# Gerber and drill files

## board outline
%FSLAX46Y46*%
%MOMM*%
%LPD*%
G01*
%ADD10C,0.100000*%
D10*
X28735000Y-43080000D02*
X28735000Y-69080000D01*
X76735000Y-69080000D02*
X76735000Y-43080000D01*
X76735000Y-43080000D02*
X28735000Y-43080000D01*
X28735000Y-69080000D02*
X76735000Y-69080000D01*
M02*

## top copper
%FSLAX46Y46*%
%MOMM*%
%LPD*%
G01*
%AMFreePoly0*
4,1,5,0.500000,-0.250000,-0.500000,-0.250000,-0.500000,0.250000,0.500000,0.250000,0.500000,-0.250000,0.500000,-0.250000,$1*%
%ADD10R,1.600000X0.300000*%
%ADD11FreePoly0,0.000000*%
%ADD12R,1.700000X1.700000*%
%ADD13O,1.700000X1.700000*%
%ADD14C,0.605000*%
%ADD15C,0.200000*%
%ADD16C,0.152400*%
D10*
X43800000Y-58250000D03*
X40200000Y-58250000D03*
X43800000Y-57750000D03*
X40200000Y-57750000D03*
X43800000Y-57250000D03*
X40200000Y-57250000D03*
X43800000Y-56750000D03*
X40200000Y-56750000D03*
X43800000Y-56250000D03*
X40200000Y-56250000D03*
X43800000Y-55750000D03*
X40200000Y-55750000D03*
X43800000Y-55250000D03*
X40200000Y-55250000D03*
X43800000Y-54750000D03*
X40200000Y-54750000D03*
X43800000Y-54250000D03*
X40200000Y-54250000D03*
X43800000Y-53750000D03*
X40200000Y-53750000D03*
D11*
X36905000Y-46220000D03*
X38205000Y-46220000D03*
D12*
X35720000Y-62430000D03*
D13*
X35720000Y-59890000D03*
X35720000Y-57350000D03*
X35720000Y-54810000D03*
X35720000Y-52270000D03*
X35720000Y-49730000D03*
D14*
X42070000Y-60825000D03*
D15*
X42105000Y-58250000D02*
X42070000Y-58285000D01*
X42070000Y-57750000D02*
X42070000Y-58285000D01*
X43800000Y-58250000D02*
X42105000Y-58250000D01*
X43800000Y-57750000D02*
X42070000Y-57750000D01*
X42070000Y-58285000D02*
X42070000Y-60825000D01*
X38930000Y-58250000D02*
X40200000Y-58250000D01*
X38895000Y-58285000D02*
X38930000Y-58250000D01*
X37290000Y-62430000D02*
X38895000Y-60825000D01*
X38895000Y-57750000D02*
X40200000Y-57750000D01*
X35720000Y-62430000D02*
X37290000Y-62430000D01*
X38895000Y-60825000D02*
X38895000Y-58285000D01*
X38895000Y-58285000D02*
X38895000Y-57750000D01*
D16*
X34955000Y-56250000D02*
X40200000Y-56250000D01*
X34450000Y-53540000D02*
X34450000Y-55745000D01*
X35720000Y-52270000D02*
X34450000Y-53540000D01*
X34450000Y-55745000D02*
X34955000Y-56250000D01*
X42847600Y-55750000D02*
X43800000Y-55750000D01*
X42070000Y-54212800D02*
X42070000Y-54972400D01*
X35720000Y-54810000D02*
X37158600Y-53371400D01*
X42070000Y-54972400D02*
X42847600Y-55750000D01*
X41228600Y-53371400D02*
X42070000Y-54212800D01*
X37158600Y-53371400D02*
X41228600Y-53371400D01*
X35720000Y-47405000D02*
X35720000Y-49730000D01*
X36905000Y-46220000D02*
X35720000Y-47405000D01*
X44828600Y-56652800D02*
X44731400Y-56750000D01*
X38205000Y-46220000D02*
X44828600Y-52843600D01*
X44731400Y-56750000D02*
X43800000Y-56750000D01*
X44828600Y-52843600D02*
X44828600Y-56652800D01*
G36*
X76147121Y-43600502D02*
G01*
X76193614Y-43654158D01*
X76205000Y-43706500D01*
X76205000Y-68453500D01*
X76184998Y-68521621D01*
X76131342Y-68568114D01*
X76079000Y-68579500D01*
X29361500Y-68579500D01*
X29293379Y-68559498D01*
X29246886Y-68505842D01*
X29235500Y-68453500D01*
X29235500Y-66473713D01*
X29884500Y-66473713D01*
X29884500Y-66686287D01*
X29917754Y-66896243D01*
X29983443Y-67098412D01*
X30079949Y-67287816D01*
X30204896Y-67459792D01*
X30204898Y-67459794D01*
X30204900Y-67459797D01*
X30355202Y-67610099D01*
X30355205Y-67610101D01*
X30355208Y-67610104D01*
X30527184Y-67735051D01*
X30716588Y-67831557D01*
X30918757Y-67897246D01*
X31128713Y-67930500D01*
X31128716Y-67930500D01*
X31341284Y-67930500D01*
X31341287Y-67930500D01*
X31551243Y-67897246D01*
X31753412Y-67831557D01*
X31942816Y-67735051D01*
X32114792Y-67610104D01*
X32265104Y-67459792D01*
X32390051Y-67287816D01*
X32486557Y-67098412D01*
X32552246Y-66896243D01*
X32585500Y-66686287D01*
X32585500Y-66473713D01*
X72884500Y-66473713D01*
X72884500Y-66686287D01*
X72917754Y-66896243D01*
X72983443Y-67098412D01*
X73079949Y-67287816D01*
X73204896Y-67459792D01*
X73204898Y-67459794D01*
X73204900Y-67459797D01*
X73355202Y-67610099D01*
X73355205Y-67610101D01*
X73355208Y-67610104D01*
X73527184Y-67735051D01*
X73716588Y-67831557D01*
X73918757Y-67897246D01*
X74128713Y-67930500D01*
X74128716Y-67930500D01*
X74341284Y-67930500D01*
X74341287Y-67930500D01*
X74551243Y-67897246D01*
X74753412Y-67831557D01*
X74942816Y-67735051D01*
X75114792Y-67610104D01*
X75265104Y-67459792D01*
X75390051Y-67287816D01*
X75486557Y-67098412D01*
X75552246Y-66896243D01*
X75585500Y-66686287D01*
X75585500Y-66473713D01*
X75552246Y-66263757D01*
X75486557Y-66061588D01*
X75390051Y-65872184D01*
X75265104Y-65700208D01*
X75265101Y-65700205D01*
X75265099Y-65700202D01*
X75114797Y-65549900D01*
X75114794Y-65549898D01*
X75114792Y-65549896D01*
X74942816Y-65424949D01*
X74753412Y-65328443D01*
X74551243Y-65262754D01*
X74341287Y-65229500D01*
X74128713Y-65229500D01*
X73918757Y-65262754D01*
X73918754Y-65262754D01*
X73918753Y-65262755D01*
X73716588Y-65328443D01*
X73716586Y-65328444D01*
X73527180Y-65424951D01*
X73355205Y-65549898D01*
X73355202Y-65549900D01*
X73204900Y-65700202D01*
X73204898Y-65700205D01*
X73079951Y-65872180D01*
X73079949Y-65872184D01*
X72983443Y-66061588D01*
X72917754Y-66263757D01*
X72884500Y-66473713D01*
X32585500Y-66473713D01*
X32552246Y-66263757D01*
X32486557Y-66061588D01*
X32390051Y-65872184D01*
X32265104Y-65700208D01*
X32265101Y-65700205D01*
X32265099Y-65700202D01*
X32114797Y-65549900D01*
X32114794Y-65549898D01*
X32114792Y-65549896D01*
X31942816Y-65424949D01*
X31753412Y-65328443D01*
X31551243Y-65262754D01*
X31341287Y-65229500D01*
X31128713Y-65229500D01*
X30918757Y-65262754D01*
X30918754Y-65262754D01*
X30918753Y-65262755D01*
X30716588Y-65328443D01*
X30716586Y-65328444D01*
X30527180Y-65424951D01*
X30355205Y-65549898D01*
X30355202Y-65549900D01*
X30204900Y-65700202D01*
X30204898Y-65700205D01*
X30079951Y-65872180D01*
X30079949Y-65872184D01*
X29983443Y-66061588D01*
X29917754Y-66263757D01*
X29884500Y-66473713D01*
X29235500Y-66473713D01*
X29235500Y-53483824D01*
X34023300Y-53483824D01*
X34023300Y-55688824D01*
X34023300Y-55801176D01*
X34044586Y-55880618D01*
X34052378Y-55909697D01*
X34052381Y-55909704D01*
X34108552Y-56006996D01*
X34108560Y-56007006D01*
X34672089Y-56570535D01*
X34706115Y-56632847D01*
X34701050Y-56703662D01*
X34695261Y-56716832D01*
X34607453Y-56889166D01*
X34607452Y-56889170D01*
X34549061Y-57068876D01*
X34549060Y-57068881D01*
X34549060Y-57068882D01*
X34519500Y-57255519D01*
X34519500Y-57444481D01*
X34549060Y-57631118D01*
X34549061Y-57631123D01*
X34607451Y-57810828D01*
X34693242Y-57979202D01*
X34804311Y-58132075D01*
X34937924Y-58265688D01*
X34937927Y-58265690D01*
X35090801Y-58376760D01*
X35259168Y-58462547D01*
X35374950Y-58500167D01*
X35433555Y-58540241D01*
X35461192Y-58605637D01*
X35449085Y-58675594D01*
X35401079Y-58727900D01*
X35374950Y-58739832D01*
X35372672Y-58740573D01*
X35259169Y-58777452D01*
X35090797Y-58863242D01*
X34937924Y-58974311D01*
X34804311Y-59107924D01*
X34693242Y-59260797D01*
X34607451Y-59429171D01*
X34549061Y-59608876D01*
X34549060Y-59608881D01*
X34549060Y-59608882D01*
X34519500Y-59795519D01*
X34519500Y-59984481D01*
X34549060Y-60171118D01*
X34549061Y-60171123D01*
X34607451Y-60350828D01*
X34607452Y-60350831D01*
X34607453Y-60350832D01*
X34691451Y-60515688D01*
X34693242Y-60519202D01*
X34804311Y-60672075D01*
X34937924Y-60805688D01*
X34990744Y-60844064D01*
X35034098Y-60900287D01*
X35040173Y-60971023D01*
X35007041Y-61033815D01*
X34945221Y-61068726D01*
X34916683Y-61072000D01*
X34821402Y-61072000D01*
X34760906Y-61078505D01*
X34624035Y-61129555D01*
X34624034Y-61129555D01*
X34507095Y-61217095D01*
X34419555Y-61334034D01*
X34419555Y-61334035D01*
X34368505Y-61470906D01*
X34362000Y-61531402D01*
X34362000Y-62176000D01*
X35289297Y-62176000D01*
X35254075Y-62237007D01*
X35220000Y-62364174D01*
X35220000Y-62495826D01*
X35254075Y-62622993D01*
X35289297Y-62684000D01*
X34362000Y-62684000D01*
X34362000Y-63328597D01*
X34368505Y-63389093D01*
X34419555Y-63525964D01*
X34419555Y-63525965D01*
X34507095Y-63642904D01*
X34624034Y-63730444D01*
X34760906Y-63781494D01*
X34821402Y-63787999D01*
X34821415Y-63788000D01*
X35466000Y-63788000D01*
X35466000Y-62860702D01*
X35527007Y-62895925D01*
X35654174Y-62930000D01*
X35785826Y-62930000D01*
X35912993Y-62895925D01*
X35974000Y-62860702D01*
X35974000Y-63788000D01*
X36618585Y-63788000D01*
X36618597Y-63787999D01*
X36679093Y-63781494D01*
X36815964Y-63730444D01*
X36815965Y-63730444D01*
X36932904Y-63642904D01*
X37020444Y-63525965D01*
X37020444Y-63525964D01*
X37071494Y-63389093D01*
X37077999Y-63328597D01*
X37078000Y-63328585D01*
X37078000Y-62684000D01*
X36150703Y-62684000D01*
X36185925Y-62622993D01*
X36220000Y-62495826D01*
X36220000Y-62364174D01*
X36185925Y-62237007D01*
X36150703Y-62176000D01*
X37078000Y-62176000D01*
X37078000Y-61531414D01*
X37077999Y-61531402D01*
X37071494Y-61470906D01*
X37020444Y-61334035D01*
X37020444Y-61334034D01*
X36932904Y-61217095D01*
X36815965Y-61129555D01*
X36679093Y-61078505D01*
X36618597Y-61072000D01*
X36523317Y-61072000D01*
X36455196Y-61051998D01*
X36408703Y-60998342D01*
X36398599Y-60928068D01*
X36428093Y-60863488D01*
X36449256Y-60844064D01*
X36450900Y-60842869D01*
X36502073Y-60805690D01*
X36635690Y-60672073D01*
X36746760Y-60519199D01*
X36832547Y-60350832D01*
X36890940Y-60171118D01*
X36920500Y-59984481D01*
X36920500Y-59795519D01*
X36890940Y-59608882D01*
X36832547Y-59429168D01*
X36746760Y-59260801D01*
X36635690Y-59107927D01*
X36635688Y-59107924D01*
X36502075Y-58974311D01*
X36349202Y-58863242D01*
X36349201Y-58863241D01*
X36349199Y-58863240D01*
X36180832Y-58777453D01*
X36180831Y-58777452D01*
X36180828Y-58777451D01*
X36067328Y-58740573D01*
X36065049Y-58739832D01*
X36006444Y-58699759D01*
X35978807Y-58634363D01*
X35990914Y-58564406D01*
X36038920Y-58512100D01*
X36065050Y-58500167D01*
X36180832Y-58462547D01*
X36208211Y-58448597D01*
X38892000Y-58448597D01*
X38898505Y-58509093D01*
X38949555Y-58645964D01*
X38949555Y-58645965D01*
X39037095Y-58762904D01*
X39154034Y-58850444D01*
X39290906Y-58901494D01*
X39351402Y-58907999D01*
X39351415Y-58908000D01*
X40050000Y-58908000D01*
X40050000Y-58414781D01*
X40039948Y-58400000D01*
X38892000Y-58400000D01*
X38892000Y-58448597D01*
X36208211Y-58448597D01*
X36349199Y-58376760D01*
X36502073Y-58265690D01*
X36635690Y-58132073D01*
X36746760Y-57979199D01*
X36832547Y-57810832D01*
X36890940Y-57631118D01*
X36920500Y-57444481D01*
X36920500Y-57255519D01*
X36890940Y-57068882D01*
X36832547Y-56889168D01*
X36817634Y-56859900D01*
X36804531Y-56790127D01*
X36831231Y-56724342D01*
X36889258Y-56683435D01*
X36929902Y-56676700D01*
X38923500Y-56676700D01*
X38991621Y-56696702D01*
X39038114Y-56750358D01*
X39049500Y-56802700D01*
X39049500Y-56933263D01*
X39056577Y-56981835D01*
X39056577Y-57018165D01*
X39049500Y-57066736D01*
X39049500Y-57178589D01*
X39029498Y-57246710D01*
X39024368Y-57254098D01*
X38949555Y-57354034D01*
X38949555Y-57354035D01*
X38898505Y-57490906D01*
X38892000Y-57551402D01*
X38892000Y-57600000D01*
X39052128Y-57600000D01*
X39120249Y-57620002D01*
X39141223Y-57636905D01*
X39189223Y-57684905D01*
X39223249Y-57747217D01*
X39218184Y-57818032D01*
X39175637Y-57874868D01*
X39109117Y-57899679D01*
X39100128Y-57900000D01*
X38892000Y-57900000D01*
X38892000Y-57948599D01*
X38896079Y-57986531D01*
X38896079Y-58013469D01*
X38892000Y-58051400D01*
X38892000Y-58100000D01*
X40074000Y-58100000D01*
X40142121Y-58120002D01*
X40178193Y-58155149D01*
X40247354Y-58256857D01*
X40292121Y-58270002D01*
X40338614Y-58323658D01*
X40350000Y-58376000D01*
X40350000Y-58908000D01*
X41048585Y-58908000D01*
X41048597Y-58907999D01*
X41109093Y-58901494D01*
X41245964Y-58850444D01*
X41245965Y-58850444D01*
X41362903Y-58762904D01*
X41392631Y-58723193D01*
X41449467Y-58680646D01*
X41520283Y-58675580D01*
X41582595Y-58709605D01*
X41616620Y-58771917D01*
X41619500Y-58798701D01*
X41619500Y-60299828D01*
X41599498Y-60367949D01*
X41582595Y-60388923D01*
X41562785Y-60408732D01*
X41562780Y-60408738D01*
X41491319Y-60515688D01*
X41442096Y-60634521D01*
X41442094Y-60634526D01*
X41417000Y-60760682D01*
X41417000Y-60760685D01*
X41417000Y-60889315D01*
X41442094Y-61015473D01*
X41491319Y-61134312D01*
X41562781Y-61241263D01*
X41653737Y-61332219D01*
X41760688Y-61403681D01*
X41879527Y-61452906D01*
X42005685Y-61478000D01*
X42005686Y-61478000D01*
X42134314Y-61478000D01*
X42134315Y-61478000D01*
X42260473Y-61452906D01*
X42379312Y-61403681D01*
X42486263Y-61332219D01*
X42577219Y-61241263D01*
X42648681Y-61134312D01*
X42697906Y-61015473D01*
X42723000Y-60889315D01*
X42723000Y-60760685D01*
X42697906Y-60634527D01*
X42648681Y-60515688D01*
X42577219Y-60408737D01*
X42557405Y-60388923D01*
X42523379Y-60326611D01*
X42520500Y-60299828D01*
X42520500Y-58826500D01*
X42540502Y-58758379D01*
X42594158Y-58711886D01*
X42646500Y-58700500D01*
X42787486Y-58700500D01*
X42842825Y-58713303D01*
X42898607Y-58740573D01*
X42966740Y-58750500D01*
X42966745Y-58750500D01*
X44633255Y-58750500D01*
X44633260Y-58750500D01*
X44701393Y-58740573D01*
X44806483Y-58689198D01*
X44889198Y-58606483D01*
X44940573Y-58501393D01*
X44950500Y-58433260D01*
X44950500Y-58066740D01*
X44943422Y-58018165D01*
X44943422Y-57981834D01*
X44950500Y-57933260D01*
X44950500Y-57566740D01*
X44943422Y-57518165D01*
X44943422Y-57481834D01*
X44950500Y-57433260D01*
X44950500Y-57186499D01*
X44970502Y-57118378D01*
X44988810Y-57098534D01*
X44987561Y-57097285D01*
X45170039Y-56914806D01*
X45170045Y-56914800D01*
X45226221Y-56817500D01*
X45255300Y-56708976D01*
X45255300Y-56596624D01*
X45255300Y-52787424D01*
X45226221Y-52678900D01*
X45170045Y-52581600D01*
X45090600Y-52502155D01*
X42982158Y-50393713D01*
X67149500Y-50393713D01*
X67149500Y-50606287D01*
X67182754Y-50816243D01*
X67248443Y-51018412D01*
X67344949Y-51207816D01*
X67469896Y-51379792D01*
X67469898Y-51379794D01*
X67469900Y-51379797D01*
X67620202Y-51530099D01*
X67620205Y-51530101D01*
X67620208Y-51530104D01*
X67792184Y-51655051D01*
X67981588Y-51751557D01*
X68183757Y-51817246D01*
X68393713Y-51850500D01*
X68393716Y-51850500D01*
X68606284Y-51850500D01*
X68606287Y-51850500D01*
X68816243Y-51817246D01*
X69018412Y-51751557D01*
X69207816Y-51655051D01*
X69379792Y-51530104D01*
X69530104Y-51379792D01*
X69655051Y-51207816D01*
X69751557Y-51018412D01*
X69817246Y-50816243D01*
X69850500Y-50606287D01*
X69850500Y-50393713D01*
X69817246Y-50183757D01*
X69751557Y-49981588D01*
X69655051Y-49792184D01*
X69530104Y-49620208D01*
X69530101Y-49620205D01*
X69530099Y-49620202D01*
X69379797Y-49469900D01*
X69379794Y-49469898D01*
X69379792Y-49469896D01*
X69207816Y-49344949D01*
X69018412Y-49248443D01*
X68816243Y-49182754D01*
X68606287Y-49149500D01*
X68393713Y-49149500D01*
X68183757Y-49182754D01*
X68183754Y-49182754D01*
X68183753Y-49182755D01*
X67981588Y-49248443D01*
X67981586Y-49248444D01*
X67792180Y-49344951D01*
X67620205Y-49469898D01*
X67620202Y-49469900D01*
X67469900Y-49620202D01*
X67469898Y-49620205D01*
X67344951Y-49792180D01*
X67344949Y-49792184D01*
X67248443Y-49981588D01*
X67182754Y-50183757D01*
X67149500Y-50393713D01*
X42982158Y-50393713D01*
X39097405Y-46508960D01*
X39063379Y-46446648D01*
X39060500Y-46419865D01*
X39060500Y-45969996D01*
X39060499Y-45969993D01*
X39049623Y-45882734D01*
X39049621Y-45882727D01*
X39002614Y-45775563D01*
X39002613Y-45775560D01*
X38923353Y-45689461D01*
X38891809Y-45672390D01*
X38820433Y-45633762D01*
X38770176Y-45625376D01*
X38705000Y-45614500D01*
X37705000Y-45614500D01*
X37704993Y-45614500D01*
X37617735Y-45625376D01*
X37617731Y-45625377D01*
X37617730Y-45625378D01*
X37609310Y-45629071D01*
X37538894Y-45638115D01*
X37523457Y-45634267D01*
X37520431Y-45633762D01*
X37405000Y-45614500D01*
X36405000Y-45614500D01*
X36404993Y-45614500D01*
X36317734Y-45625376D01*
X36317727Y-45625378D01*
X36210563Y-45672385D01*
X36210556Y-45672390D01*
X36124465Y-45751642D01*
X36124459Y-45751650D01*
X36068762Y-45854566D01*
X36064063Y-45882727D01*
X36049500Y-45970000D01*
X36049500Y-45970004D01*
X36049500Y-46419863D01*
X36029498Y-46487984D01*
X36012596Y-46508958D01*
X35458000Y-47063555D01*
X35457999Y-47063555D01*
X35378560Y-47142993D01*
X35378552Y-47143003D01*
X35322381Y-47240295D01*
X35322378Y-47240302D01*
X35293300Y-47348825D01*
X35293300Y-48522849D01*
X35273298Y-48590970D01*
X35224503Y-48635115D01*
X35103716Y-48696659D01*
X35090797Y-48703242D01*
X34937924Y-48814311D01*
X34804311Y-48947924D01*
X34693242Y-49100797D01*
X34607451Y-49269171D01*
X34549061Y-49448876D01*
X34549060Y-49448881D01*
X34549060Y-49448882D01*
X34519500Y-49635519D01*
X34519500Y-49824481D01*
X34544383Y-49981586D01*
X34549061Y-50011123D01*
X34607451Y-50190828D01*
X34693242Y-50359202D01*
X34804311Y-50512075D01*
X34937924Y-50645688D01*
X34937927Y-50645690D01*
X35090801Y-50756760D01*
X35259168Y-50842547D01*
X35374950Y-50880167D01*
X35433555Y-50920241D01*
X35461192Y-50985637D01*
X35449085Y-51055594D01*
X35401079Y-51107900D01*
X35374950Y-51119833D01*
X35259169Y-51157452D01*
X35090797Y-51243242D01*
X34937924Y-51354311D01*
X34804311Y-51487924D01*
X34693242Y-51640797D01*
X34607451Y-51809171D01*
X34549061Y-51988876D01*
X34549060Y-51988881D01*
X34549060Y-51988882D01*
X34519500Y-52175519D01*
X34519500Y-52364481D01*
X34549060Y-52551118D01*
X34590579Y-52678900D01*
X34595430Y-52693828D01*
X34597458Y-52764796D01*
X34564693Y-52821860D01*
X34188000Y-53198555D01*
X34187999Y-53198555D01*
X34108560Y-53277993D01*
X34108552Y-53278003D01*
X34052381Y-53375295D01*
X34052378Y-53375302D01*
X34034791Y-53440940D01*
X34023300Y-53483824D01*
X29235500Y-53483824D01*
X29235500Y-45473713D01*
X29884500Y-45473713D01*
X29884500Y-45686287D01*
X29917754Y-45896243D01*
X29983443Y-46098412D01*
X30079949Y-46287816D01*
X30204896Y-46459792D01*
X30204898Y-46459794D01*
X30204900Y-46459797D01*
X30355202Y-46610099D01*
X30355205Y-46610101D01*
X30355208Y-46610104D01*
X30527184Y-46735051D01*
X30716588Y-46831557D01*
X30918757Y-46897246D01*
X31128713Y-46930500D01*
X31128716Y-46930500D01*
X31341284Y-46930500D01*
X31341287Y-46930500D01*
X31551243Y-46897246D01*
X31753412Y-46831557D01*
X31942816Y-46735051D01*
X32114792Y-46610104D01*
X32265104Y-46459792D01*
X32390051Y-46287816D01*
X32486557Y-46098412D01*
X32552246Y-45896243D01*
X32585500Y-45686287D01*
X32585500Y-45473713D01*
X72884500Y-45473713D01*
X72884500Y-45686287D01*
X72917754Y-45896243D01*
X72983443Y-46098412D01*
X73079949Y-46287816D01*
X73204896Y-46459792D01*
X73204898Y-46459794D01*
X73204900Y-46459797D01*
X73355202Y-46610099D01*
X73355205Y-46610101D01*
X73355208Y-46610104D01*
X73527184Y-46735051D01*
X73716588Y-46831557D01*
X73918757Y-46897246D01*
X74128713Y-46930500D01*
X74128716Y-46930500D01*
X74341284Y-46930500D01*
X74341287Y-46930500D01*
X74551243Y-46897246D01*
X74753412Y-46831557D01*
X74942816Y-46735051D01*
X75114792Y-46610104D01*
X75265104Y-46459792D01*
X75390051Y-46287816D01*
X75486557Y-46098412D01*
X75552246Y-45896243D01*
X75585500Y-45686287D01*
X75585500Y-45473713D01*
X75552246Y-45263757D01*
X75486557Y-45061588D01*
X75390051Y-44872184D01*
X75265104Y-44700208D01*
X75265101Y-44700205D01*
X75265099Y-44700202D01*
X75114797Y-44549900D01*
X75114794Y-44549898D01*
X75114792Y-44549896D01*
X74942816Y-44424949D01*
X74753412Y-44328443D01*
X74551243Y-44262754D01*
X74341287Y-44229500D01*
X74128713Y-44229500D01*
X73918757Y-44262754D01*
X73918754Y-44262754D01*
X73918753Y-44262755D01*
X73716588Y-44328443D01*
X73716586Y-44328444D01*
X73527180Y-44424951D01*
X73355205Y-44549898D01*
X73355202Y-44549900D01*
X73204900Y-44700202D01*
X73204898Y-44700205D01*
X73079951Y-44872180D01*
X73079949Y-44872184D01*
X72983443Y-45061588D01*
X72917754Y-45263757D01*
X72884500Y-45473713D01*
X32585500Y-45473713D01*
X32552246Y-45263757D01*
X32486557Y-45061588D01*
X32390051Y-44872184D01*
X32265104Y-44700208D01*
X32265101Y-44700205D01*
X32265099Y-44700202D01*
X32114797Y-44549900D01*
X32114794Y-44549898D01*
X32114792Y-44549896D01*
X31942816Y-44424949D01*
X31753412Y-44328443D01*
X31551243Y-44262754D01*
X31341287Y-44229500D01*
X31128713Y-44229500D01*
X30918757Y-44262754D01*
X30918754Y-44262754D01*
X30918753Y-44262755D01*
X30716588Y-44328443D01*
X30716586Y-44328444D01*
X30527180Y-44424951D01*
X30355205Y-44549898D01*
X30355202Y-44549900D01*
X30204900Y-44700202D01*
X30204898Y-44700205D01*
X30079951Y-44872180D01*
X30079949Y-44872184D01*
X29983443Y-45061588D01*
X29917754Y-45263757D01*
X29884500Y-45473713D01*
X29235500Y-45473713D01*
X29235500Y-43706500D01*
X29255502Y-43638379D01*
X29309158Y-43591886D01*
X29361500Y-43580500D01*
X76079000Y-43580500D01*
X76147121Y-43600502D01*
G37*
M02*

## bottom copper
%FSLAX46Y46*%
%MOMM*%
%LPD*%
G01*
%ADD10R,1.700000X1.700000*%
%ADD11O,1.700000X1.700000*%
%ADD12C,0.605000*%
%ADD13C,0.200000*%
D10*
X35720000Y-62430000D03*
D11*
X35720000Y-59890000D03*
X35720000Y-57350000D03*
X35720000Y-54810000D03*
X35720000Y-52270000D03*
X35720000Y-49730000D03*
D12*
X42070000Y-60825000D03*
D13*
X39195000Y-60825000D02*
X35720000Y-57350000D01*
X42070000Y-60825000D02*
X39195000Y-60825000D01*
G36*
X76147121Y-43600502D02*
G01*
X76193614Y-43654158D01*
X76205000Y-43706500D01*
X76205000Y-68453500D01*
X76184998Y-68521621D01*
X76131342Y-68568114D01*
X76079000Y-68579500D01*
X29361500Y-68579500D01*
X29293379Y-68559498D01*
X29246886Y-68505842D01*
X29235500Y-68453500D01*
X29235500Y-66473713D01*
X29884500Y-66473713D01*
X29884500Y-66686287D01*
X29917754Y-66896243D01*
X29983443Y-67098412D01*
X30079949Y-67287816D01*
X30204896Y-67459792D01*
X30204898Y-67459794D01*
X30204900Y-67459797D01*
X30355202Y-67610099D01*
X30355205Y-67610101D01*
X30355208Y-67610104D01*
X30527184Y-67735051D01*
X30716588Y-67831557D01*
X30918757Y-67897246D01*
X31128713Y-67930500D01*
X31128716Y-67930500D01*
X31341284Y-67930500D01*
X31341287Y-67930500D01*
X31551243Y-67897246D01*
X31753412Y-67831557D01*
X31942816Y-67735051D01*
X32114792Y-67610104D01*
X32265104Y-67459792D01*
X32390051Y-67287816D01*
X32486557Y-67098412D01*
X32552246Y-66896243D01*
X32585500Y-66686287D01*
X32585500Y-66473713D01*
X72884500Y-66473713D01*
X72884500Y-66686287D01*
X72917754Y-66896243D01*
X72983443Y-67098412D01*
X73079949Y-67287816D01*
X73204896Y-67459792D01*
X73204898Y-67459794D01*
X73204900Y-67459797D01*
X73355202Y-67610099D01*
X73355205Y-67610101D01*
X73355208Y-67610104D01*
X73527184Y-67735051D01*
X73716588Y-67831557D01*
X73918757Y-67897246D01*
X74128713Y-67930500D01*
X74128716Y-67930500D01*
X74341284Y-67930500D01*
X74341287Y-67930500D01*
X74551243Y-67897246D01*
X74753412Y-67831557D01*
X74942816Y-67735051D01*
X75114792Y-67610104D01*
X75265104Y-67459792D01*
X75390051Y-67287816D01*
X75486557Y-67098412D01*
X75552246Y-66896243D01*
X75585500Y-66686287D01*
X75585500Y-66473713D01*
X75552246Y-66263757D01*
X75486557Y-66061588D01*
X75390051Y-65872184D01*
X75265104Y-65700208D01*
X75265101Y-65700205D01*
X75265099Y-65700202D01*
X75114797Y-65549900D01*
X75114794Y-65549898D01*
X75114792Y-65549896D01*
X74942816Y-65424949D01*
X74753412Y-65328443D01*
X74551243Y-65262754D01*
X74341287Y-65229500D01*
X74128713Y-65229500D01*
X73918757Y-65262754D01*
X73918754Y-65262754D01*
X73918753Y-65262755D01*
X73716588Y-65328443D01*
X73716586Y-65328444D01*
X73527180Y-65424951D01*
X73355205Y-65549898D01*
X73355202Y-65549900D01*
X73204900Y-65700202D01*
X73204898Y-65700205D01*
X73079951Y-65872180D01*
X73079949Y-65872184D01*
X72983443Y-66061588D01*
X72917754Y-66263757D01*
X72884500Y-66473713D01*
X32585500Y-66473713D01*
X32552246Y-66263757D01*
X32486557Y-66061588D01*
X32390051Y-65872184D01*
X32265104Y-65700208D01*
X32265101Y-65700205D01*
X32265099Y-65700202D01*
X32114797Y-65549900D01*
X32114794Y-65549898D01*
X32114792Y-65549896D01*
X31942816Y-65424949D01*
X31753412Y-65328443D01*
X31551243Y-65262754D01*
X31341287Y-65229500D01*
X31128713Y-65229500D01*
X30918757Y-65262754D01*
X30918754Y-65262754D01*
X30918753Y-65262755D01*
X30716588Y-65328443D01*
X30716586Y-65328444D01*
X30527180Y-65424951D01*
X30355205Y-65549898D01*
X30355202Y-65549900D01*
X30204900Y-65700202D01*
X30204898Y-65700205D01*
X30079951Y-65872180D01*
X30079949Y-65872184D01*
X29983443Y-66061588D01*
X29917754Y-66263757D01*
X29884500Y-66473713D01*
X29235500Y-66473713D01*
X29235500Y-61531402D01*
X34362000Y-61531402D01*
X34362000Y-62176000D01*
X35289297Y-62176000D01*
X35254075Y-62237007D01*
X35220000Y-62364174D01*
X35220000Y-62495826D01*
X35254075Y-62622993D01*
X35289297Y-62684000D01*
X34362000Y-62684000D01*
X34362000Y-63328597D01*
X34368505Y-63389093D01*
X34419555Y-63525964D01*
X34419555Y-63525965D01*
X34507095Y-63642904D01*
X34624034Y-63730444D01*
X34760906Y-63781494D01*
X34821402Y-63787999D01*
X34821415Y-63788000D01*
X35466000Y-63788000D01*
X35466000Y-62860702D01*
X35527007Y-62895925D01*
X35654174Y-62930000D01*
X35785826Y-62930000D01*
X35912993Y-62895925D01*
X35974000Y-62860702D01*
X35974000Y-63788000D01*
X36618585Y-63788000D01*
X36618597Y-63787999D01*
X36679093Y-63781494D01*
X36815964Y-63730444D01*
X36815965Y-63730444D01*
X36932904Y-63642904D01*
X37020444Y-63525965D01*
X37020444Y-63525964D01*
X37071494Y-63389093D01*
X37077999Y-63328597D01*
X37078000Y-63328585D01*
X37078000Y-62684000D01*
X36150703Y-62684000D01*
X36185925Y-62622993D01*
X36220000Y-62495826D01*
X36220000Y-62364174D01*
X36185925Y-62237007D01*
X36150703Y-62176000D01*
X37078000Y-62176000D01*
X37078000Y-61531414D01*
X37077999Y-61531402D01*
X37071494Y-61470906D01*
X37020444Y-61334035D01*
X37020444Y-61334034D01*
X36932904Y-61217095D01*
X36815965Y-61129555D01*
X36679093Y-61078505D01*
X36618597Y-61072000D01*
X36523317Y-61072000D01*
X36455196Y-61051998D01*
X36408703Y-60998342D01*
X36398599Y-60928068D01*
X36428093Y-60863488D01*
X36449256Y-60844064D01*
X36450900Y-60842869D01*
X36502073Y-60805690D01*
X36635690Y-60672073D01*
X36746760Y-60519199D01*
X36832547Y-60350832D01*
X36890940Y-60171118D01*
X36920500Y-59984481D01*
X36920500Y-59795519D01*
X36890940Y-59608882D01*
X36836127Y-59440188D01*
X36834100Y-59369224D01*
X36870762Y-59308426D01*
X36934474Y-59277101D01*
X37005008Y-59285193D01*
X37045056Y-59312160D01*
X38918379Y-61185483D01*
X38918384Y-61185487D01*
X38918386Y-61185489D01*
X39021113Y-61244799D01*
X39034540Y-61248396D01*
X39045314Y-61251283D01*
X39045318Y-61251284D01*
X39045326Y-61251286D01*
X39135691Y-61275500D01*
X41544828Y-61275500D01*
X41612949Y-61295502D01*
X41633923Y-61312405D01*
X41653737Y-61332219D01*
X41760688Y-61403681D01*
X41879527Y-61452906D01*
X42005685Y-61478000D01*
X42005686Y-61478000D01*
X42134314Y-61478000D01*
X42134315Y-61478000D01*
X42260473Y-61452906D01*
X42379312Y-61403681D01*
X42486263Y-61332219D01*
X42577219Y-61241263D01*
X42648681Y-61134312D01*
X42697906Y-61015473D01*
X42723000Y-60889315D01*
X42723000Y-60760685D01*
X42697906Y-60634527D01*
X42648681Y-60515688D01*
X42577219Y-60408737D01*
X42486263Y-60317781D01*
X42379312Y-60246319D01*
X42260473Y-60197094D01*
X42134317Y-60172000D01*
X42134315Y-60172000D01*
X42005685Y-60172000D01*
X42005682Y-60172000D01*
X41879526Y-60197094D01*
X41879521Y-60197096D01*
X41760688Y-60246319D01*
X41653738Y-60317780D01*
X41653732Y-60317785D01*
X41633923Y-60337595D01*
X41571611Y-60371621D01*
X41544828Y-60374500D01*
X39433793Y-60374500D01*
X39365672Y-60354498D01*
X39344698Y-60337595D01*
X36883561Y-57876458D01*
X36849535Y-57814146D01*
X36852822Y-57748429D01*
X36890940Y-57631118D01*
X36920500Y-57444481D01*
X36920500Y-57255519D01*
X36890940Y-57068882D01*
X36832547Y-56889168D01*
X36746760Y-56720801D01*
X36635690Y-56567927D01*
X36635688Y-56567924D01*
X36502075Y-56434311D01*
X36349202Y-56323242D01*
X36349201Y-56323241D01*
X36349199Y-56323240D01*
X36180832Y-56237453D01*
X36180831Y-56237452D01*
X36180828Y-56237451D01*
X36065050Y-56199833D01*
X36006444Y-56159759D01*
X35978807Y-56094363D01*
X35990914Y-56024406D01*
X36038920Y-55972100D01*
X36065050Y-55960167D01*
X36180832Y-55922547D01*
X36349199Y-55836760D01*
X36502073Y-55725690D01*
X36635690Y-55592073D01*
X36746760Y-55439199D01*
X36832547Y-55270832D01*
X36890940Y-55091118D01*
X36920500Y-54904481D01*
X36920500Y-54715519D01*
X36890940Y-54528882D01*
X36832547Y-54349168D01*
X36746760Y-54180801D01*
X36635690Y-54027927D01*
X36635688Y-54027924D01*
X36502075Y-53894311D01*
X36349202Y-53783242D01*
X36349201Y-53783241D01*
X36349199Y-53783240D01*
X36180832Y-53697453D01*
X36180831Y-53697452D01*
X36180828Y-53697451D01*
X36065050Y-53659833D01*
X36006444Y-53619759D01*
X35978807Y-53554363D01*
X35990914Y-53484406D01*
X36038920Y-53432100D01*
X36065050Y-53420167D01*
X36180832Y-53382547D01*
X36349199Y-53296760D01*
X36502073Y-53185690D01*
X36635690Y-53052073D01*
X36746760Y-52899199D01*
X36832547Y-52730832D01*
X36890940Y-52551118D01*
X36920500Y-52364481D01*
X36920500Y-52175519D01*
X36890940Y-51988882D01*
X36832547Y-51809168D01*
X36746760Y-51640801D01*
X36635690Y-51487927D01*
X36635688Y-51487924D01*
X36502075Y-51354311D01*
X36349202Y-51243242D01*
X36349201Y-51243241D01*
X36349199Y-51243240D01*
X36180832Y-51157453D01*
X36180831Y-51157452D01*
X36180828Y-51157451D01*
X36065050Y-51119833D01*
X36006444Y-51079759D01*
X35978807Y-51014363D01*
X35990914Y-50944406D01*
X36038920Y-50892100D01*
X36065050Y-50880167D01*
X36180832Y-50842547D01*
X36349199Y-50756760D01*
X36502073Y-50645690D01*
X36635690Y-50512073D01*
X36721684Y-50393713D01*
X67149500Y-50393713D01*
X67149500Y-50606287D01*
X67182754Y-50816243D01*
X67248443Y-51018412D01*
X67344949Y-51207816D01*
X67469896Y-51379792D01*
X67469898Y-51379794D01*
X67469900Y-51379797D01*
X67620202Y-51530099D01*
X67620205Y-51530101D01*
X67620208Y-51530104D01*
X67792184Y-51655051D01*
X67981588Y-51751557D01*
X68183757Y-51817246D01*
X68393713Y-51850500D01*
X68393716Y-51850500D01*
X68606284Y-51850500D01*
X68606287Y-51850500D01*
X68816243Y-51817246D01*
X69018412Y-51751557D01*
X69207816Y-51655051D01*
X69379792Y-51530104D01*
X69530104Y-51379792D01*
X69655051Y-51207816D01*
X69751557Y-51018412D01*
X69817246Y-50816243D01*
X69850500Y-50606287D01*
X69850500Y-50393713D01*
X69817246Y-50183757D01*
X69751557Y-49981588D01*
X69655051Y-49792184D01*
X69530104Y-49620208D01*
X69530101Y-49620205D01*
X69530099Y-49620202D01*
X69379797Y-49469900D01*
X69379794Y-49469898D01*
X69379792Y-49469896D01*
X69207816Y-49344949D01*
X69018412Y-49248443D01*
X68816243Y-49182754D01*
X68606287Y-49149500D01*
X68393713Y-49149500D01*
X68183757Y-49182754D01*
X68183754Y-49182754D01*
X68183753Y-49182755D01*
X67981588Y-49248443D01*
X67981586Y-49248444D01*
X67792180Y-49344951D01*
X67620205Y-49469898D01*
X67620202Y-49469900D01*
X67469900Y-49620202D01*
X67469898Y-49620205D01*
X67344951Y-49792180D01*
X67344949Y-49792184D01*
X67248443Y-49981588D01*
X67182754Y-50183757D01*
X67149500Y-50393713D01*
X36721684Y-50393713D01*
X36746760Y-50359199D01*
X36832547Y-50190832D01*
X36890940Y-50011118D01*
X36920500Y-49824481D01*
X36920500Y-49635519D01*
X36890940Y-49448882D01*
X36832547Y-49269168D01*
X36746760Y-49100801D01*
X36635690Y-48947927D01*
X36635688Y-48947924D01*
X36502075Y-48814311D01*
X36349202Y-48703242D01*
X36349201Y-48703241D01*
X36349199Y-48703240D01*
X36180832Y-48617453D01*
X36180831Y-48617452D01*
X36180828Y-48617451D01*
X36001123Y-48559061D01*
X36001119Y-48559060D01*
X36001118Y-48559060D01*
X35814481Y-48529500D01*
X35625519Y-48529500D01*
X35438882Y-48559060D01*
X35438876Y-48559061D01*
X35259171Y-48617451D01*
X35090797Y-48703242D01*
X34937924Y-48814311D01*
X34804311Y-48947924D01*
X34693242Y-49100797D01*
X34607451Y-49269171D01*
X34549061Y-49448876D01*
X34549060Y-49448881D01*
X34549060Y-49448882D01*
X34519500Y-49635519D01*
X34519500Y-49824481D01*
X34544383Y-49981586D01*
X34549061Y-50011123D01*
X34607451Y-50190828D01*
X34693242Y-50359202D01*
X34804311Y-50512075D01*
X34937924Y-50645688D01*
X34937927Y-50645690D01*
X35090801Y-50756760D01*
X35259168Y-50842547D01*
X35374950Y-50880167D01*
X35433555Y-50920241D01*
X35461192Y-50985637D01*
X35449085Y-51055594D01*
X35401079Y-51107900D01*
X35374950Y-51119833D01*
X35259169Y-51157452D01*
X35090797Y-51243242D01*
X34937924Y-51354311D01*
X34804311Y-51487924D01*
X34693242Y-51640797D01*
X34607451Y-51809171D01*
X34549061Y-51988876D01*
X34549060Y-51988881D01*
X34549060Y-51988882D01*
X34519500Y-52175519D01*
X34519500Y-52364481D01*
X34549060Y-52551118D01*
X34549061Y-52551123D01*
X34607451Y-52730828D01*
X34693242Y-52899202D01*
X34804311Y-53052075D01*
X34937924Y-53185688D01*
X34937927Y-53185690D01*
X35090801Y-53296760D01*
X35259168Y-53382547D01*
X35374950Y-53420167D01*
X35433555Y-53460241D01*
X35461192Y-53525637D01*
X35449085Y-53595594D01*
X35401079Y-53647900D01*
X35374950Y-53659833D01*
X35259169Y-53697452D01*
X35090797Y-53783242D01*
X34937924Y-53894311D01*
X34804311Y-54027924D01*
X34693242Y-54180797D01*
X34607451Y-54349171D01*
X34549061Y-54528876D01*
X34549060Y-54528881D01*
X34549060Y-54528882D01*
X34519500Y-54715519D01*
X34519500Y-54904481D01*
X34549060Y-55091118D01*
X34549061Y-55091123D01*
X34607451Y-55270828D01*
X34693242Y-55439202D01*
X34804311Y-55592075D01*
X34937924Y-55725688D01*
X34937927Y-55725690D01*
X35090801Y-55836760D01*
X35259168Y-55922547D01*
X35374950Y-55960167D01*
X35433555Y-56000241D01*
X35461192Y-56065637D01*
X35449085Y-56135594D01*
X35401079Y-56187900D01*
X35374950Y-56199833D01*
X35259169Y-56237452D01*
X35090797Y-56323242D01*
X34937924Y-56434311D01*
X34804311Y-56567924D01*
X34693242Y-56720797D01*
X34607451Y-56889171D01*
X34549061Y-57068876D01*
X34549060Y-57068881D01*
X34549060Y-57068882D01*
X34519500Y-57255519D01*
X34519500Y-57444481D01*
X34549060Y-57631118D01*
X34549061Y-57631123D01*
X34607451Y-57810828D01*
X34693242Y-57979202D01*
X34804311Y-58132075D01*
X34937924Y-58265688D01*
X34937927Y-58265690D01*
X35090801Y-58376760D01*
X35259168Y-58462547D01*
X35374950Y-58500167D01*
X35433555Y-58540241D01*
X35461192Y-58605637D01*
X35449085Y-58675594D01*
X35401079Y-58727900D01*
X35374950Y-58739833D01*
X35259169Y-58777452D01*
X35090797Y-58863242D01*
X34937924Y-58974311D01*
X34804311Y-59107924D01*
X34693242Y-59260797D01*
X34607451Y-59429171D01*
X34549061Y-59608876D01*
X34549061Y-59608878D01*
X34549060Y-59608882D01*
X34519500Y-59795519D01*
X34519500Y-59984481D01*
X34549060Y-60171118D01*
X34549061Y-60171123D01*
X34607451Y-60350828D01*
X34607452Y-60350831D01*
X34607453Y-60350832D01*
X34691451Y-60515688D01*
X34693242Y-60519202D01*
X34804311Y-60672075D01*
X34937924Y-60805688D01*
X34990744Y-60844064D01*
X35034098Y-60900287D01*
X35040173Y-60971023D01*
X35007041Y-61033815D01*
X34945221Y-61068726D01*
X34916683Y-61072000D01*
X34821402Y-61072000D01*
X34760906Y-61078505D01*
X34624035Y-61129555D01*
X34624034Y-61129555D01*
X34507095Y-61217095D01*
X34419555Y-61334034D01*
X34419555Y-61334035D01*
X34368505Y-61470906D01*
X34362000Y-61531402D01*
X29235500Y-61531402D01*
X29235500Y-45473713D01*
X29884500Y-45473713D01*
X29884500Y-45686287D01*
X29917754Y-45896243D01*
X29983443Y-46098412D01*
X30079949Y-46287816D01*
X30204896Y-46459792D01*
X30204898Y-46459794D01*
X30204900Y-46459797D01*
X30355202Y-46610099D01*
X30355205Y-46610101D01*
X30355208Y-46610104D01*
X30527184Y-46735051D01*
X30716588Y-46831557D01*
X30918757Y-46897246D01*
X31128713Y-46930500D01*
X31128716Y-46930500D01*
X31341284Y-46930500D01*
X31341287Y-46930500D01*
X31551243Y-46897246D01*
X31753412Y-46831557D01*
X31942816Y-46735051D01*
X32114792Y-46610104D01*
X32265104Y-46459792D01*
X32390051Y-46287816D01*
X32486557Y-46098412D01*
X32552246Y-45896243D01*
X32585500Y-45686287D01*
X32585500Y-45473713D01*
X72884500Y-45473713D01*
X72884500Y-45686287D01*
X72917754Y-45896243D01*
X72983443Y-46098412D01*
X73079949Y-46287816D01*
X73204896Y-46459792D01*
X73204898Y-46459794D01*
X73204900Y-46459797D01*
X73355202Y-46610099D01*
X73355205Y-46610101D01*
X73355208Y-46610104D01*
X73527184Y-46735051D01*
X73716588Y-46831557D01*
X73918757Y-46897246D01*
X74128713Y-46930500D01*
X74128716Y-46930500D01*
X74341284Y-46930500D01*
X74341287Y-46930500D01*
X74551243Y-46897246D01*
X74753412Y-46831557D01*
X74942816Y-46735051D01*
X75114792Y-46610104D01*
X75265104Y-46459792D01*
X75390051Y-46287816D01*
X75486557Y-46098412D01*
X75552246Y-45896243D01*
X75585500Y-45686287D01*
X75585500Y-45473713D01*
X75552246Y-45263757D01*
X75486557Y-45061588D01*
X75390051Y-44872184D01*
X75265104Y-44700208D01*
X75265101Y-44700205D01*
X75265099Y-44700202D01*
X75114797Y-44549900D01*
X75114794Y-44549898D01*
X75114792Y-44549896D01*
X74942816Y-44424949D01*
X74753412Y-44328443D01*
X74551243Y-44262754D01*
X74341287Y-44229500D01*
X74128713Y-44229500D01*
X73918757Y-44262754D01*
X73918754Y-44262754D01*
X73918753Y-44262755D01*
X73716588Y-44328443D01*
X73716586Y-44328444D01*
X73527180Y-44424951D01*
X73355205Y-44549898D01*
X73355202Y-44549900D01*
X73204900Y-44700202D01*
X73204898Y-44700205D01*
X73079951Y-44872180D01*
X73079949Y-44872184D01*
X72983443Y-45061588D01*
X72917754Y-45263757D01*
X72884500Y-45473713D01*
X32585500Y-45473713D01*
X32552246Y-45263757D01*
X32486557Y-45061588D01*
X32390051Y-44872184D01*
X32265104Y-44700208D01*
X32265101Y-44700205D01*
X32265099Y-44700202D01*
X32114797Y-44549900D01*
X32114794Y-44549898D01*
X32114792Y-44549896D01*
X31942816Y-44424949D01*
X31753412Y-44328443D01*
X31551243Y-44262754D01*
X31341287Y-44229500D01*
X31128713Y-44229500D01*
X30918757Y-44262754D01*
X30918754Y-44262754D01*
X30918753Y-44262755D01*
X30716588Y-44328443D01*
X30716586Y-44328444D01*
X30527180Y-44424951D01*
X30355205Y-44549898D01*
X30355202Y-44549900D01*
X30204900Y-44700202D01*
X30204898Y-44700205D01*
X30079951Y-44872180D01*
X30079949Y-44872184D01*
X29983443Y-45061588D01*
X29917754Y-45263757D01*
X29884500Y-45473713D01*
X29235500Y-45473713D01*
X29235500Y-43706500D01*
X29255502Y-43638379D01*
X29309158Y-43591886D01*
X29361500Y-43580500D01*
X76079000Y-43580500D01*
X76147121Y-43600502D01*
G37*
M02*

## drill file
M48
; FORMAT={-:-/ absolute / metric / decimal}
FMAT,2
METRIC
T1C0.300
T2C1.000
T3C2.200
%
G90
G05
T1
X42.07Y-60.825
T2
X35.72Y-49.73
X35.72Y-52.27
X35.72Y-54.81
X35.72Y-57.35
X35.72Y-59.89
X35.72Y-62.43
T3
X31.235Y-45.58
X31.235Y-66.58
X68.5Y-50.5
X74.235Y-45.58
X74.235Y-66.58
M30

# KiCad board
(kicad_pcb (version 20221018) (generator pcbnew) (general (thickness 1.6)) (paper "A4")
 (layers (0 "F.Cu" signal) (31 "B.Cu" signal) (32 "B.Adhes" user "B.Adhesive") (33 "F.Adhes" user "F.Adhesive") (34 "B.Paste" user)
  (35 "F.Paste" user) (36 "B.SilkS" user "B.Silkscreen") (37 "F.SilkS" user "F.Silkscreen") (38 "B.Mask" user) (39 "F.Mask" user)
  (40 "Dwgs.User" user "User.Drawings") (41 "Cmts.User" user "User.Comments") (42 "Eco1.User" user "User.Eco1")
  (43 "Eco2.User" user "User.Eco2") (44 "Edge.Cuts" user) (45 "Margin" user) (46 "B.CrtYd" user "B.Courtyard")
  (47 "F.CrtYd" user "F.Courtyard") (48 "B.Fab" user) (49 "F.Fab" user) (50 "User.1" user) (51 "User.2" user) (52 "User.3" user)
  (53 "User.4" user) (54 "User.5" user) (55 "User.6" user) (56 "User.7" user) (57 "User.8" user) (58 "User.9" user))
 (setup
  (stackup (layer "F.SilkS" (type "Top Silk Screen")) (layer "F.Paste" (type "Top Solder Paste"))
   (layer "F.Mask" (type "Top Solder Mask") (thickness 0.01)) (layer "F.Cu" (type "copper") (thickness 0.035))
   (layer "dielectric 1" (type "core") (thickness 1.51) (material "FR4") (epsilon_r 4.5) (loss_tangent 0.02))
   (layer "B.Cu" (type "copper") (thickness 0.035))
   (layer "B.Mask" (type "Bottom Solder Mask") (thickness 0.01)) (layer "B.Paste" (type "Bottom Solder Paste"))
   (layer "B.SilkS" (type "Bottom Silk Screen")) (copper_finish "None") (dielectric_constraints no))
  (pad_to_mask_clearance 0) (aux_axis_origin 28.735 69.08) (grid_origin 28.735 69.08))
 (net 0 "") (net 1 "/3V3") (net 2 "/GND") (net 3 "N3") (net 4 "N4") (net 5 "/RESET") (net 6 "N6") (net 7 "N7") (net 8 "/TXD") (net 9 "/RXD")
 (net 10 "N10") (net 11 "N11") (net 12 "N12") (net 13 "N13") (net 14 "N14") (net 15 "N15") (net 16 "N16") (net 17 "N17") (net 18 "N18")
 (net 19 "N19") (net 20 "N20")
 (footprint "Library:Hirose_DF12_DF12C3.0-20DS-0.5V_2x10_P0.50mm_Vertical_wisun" (layer "F.Cu") (at 42 56 -90)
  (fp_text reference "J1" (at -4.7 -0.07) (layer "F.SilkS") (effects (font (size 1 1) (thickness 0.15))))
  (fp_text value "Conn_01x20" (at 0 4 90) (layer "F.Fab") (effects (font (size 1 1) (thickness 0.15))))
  (pad "" smd rect (at -2.25 -2 270) (size 0.28 1.2) (layers "F.Paste"))
  (pad "" smd rect (at -2.25 2 270) (size 0.28 1.2) (layers "F.Paste"))
  (pad "" smd rect (at -1.75 -2 270) (size 0.28 1.2) (layers "F.Paste"))
  (pad "" smd rect (at -1.75 2 270) (size 0.28 1.2) (layers "F.Paste"))
  (pad "" smd rect (at -1.25 -2 270) (size 0.28 1.2) (layers "F.Paste"))
  (pad "" smd rect (at -1.25 2 270) (size 0.28 1.2) (layers "F.Paste"))
  (pad "" smd rect (at -0.75 -2 270) (size 0.28 1.2) (layers "F.Paste"))
  (pad "" smd rect (at -0.75 2 270) (size 0.28 1.2) (layers "F.Paste"))
  (pad "" smd rect (at -0.25 -2 270) (size 0.28 1.2) (layers "F.Paste"))
  (pad "" smd rect (at -0.25 2 270) (size 0.28 1.2) (layers "F.Paste"))
  (pad "" smd rect (at 0.25 -2 270) (size 0.28 1.2) (layers "F.Paste"))
  (pad "" smd rect (at 0.25 2 270) (size 0.28 1.2) (layers "F.Paste"))
  (pad "" smd rect (at 0.75 -2 270) (size 0.28 1.2) (layers "F.Paste"))
  (pad "" smd rect (at 0.75 2 270) (size 0.28 1.2) (layers "F.Paste"))
  (pad "" smd rect (at 1.25 -2 270) (size 0.28 1.2) (layers "F.Paste"))
  (pad "" smd rect (at 1.25 2 270) (size 0.28 1.2) (layers "F.Paste"))
  (pad "" smd rect (at 1.75 -2 270) (size 0.28 1.2) (layers "F.Paste"))
  (pad "" smd rect (at 1.75 2 270) (size 0.28 1.2) (layers "F.Paste"))
  (pad "" smd rect (at 2.25 -2 270) (size 0.28 1.2) (layers "F.Paste"))
  (pad "" smd rect (at 2.25 2 270) (size 0.28 1.2) (layers "F.Paste"))
  (pad "1" smd rect (at 2.25 -1.8 270) (size 0.3 1.6) (layers "F.Cu" "F.Mask") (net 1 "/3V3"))
  (pad "2" smd rect (at 2.25 1.8 270) (size 0.3 1.6) (layers "F.Cu" "F.Mask") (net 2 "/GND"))
  (pad "3" smd rect (at 1.75 -1.8 270) (size 0.3 1.6) (layers "F.Cu" "F.Mask") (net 1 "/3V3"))
  (pad "4" smd rect (at 1.75 1.8 270) (size 0.3 1.6) (layers "F.Cu" "F.Mask") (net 2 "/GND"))
  (pad "5" smd rect (at 1.25 -1.8 270) (size 0.3 1.6) (layers "F.Cu" "F.Mask") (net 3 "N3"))
  (pad "6" smd rect (at 1.25 1.8 270) (size 0.3 1.6) (layers "F.Cu" "F.Mask") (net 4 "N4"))
  (pad "7" smd rect (at 0.75 -1.8 270) (size 0.3 1.6) (layers "F.Cu" "F.Mask") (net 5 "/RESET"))
  (pad "8" smd rect (at 0.75 1.8 270) (size 0.3 1.6) (layers "F.Cu" "F.Mask") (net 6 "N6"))
  (pad "9" smd rect (at 0.25 -1.8 270) (size 0.3 1.6) (layers "F.Cu" "F.Mask") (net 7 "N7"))
  (pad "10" smd rect (at 0.25 1.8 270) (size 0.3 1.6) (layers "F.Cu" "F.Mask") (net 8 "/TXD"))
  (pad "11" smd rect (at -0.25 -1.8 270) (size 0.3 1.6) (layers "F.Cu" "F.Mask") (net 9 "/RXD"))
  (pad "12" smd rect (at -0.25 1.8 270) (size 0.3 1.6) (layers "F.Cu" "F.Mask") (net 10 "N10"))
  (pad "13" smd rect (at -0.75 -1.8 270) (size 0.3 1.6) (layers "F.Cu" "F.Mask") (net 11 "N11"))
  (pad "14" smd rect (at -0.75 1.8 270) (size 0.3 1.6) (layers "F.Cu" "F.Mask") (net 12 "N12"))
  (pad "15" smd rect (at -1.25 -1.8 270) (size 0.3 1.6) (layers "F.Cu" "F.Mask") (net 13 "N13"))
  (pad "16" smd rect (at -1.25 1.8 270) (size 0.3 1.6) (layers "F.Cu" "F.Mask") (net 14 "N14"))
  (pad "17" smd rect (at -1.75 -1.8 270) (size 0.3 1.6) (layers "F.Cu" "F.Mask") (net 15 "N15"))
  (pad "18" smd rect (at -1.75 1.8 270) (size 0.3 1.6) (layers "F.Cu" "F.Mask") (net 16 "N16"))
  (pad "19" smd rect (at -2.25 -1.8 270) (size 0.3 1.6) (layers "F.Cu" "F.Mask") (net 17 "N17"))
  (pad "20" smd rect (at -2.25 1.8 270) (size 0.3 1.6) (layers "F.Cu" "F.Mask") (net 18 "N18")))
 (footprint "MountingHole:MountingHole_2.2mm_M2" (layer "F.Cu") (at 68.5 50.5)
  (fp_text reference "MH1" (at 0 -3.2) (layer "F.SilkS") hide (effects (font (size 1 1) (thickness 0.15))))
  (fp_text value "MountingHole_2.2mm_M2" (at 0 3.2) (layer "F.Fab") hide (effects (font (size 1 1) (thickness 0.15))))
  (pad "" np_thru_hole circle (at 0 0) (size 2.2 2.2) (drill 2.2) (layers "*.Cu" "*.Mask")))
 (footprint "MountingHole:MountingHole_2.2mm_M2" (layer "F.Cu") (at 31.235 45.58)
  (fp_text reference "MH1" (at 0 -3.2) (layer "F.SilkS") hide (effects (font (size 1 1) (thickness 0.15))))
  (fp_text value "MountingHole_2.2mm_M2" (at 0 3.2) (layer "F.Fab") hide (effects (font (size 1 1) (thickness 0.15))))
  (pad "" np_thru_hole circle (at 0 0) (size 2.2 2.2) (drill 2.2) (layers "F&B.Cu" "*.Mask")))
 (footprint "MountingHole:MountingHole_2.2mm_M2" (layer "F.Cu") (at 74.235 45.58)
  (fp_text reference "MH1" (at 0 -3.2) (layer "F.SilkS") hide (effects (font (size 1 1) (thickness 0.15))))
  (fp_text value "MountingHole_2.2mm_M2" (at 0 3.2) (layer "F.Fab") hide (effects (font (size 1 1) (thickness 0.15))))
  (pad "" np_thru_hole circle (at 0 0) (size 2.2 2.2) (drill 2.2) (layers "F&B.Cu" "*.Mask")))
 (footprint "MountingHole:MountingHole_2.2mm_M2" (layer "F.Cu") (at 31.235 66.58)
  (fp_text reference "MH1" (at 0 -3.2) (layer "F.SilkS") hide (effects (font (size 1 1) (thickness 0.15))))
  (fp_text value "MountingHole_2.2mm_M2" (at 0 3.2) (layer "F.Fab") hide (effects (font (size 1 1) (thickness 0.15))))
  (pad "" np_thru_hole circle (at 0 0) (size 2.2 2.2) (drill 2.2) (layers "F&B.Cu" "*.Mask")))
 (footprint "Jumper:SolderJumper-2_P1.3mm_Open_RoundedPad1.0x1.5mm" (layer "F.Cu") (at 37.555 46.22)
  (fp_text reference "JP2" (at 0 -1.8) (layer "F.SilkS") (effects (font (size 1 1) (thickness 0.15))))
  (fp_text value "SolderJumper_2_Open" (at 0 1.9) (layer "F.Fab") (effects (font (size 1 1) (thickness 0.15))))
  (pad "1" smd custom (at -0.65 0) (size 1 0.5) (layers "F.Cu" "F.Mask") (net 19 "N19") (zone_connect 2) (thermal_bridge_angle 45)
   (options (clearance outline) (anchor rect)) (primitives))
  (pad "2" smd custom (at 0.65 0) (size 1 0.5) (layers "F.Cu" "F.Mask") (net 5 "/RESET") (zone_connect 2) (thermal_bridge_angle 45)
   (options (clearance outline) (anchor rect)) (primitives)))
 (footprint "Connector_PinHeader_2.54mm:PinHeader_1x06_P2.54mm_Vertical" (layer "F.Cu") (at 35.72 62.43 180)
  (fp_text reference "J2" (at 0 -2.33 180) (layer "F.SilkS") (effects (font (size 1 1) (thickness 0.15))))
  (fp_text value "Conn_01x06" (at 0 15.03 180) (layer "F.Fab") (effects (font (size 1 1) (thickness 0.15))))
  (pad "1" thru_hole rect (at 0 0 180) (size 1.7 1.7) (drill 1) (layers "*.Cu" "*.Mask") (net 2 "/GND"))
  (pad "2" thru_hole oval (at 0 2.54 180) (size 1.7 1.7) (drill 1) (layers "*.Cu" "*.Mask") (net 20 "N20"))
  (pad "3" thru_hole oval (at 0 5.08 180) (size 1.7 1.7) (drill 1) (layers "*.Cu" "*.Mask") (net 1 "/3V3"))
  (pad "4" thru_hole oval (at 0 7.62 180) (size 1.7 1.7) (drill 1) (layers "*.Cu" "*.Mask") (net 9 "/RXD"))
  (pad "5" thru_hole oval (at 0 10.16 180) (size 1.7 1.7) (drill 1) (layers "*.Cu" "*.Mask") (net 8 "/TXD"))
  (pad "6" thru_hole oval (at 0 12.7 180) (size 1.7 1.7) (drill 1) (layers "*.Cu" "*.Mask") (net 19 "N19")))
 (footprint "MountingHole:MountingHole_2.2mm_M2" (layer "F.Cu") (at 74.235 66.58)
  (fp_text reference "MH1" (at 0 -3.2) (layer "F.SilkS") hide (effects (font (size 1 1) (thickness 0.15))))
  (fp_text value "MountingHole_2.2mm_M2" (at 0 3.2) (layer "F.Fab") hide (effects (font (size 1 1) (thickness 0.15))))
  (pad "" np_thru_hole circle (at 0 0) (size 2.2 2.2) (drill 2.2) (layers "F&B.Cu" "*.Mask")))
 (gr_line (start 28.735 43.08) (end 28.735 69.08) (stroke (width 0.1) (type default)) (layer "Edge.Cuts"))
 (gr_line (start 76.735 69.08) (end 76.735 43.08) (stroke (width 0.1) (type default)) (layer "Edge.Cuts"))
 (gr_line (start 76.735 43.08) (end 28.735 43.08) (stroke (width 0.1) (type default)) (layer "Edge.Cuts"))
 (gr_line (start 28.735 69.08) (end 76.735 69.08) (stroke (width 0.1) (type default)) (layer "Edge.Cuts"))
 (segment (start 42.105 58.25) (end 42.07 58.285) (width 0.2) (layer "F.Cu") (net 1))
 (segment (start 42.07 57.75) (end 42.07 58.285) (width 0.2) (layer "F.Cu") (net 1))
 (segment (start 43.8 58.25) (end 42.105 58.25) (width 0.2) (layer "F.Cu") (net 1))
 (segment (start 43.8 57.75) (end 42.07 57.75) (width 0.2) (layer "F.Cu") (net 1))
 (segment (start 42.07 58.285) (end 42.07 60.825) (width 0.2) (layer "F.Cu") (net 1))
 (via (at 42.07 60.825) (size 0.605) (drill 0.3) (layers "F.Cu" "B.Cu") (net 1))
 (segment (start 39.195 60.825) (end 35.72 57.35) (width 0.2) (layer "B.Cu") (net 1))
 (segment (start 42.07 60.825) (end 39.195 60.825) (width 0.2) (layer "B.Cu") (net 1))
 (segment (start 38.93 58.25) (end 40.2 58.25) (width 0.2) (layer "F.Cu") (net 2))
 (segment (start 38.895 58.285) (end 38.93 58.25) (width 0.2) (layer "F.Cu") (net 2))
 (segment (start 37.29 62.43) (end 38.895 60.825) (width 0.2) (layer "F.Cu") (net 2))
 (segment (start 38.895 57.75) (end 40.2 57.75) (width 0.2) (layer "F.Cu") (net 2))
 (segment (start 35.72 62.43) (end 37.29 62.43) (width 0.2) (layer "F.Cu") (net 2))
 (segment (start 38.895 60.825) (end 38.895 58.285) (width 0.2) (layer "F.Cu") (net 2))
 (segment (start 38.895 58.285) (end 38.895 57.75) (width 0.2) (layer "F.Cu") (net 2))
 (segment (start 34.955 56.25) (end 40.2 56.25) (width 0.1524) (layer "F.Cu") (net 8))
 (segment (start 34.45 53.54) (end 34.45 55.745) (width 0.1524) (layer "F.Cu") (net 8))
 (segment (start 35.72 52.27) (end 34.45 53.54) (width 0.1524) (layer "F.Cu") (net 8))
 (segment (start 34.45 55.745) (end 34.955 56.25) (width 0.1524) (layer "F.Cu") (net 8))
 (segment (start 42.8476 55.75) (end 43.8 55.75) (width 0.1524) (layer "F.Cu") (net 9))
 (segment (start 42.07 54.2128) (end 42.07 54.9724) (width 0.1524) (layer "F.Cu") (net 9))
 (segment (start 35.72 54.81) (end 37.1586 53.3714) (width 0.1524) (layer "F.Cu") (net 9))
 (segment (start 42.07 54.9724) (end 42.8476 55.75) (width 0.1524) (layer "F.Cu") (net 9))
 (segment (start 41.2286 53.3714) (end 42.07 54.2128) (width 0.1524) (layer "F.Cu") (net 9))
 (segment (start 37.1586 53.3714) (end 41.2286 53.3714) (width 0.1524) (layer "F.Cu") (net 9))
 (segment (start 35.72 47.405) (end 35.72 49.73) (width 0.1524) (layer "F.Cu") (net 19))
 (segment (start 36.905 46.22) (end 35.72 47.405) (width 0.1524) (layer "F.Cu") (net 19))
 (segment (start 44.8286 56.6528) (end 44.7314 56.75) (width 0.1524) (layer "F.Cu") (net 5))
 (segment (start 38.205 46.22) (end 44.8286 52.8436) (width 0.1524) (layer "F.Cu") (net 5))
 (segment (start 44.7314 56.75) (end 43.8 56.75) (width 0.1524) (layer "F.Cu") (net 5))
 (segment (start 44.8286 52.8436) (end 44.8286 56.6528) (width 0.1524) (layer "F.Cu") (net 5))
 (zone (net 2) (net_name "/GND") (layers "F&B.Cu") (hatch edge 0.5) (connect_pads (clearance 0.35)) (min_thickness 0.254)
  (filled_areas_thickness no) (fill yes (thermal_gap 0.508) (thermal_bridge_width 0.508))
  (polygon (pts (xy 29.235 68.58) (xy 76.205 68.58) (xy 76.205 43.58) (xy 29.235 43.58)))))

